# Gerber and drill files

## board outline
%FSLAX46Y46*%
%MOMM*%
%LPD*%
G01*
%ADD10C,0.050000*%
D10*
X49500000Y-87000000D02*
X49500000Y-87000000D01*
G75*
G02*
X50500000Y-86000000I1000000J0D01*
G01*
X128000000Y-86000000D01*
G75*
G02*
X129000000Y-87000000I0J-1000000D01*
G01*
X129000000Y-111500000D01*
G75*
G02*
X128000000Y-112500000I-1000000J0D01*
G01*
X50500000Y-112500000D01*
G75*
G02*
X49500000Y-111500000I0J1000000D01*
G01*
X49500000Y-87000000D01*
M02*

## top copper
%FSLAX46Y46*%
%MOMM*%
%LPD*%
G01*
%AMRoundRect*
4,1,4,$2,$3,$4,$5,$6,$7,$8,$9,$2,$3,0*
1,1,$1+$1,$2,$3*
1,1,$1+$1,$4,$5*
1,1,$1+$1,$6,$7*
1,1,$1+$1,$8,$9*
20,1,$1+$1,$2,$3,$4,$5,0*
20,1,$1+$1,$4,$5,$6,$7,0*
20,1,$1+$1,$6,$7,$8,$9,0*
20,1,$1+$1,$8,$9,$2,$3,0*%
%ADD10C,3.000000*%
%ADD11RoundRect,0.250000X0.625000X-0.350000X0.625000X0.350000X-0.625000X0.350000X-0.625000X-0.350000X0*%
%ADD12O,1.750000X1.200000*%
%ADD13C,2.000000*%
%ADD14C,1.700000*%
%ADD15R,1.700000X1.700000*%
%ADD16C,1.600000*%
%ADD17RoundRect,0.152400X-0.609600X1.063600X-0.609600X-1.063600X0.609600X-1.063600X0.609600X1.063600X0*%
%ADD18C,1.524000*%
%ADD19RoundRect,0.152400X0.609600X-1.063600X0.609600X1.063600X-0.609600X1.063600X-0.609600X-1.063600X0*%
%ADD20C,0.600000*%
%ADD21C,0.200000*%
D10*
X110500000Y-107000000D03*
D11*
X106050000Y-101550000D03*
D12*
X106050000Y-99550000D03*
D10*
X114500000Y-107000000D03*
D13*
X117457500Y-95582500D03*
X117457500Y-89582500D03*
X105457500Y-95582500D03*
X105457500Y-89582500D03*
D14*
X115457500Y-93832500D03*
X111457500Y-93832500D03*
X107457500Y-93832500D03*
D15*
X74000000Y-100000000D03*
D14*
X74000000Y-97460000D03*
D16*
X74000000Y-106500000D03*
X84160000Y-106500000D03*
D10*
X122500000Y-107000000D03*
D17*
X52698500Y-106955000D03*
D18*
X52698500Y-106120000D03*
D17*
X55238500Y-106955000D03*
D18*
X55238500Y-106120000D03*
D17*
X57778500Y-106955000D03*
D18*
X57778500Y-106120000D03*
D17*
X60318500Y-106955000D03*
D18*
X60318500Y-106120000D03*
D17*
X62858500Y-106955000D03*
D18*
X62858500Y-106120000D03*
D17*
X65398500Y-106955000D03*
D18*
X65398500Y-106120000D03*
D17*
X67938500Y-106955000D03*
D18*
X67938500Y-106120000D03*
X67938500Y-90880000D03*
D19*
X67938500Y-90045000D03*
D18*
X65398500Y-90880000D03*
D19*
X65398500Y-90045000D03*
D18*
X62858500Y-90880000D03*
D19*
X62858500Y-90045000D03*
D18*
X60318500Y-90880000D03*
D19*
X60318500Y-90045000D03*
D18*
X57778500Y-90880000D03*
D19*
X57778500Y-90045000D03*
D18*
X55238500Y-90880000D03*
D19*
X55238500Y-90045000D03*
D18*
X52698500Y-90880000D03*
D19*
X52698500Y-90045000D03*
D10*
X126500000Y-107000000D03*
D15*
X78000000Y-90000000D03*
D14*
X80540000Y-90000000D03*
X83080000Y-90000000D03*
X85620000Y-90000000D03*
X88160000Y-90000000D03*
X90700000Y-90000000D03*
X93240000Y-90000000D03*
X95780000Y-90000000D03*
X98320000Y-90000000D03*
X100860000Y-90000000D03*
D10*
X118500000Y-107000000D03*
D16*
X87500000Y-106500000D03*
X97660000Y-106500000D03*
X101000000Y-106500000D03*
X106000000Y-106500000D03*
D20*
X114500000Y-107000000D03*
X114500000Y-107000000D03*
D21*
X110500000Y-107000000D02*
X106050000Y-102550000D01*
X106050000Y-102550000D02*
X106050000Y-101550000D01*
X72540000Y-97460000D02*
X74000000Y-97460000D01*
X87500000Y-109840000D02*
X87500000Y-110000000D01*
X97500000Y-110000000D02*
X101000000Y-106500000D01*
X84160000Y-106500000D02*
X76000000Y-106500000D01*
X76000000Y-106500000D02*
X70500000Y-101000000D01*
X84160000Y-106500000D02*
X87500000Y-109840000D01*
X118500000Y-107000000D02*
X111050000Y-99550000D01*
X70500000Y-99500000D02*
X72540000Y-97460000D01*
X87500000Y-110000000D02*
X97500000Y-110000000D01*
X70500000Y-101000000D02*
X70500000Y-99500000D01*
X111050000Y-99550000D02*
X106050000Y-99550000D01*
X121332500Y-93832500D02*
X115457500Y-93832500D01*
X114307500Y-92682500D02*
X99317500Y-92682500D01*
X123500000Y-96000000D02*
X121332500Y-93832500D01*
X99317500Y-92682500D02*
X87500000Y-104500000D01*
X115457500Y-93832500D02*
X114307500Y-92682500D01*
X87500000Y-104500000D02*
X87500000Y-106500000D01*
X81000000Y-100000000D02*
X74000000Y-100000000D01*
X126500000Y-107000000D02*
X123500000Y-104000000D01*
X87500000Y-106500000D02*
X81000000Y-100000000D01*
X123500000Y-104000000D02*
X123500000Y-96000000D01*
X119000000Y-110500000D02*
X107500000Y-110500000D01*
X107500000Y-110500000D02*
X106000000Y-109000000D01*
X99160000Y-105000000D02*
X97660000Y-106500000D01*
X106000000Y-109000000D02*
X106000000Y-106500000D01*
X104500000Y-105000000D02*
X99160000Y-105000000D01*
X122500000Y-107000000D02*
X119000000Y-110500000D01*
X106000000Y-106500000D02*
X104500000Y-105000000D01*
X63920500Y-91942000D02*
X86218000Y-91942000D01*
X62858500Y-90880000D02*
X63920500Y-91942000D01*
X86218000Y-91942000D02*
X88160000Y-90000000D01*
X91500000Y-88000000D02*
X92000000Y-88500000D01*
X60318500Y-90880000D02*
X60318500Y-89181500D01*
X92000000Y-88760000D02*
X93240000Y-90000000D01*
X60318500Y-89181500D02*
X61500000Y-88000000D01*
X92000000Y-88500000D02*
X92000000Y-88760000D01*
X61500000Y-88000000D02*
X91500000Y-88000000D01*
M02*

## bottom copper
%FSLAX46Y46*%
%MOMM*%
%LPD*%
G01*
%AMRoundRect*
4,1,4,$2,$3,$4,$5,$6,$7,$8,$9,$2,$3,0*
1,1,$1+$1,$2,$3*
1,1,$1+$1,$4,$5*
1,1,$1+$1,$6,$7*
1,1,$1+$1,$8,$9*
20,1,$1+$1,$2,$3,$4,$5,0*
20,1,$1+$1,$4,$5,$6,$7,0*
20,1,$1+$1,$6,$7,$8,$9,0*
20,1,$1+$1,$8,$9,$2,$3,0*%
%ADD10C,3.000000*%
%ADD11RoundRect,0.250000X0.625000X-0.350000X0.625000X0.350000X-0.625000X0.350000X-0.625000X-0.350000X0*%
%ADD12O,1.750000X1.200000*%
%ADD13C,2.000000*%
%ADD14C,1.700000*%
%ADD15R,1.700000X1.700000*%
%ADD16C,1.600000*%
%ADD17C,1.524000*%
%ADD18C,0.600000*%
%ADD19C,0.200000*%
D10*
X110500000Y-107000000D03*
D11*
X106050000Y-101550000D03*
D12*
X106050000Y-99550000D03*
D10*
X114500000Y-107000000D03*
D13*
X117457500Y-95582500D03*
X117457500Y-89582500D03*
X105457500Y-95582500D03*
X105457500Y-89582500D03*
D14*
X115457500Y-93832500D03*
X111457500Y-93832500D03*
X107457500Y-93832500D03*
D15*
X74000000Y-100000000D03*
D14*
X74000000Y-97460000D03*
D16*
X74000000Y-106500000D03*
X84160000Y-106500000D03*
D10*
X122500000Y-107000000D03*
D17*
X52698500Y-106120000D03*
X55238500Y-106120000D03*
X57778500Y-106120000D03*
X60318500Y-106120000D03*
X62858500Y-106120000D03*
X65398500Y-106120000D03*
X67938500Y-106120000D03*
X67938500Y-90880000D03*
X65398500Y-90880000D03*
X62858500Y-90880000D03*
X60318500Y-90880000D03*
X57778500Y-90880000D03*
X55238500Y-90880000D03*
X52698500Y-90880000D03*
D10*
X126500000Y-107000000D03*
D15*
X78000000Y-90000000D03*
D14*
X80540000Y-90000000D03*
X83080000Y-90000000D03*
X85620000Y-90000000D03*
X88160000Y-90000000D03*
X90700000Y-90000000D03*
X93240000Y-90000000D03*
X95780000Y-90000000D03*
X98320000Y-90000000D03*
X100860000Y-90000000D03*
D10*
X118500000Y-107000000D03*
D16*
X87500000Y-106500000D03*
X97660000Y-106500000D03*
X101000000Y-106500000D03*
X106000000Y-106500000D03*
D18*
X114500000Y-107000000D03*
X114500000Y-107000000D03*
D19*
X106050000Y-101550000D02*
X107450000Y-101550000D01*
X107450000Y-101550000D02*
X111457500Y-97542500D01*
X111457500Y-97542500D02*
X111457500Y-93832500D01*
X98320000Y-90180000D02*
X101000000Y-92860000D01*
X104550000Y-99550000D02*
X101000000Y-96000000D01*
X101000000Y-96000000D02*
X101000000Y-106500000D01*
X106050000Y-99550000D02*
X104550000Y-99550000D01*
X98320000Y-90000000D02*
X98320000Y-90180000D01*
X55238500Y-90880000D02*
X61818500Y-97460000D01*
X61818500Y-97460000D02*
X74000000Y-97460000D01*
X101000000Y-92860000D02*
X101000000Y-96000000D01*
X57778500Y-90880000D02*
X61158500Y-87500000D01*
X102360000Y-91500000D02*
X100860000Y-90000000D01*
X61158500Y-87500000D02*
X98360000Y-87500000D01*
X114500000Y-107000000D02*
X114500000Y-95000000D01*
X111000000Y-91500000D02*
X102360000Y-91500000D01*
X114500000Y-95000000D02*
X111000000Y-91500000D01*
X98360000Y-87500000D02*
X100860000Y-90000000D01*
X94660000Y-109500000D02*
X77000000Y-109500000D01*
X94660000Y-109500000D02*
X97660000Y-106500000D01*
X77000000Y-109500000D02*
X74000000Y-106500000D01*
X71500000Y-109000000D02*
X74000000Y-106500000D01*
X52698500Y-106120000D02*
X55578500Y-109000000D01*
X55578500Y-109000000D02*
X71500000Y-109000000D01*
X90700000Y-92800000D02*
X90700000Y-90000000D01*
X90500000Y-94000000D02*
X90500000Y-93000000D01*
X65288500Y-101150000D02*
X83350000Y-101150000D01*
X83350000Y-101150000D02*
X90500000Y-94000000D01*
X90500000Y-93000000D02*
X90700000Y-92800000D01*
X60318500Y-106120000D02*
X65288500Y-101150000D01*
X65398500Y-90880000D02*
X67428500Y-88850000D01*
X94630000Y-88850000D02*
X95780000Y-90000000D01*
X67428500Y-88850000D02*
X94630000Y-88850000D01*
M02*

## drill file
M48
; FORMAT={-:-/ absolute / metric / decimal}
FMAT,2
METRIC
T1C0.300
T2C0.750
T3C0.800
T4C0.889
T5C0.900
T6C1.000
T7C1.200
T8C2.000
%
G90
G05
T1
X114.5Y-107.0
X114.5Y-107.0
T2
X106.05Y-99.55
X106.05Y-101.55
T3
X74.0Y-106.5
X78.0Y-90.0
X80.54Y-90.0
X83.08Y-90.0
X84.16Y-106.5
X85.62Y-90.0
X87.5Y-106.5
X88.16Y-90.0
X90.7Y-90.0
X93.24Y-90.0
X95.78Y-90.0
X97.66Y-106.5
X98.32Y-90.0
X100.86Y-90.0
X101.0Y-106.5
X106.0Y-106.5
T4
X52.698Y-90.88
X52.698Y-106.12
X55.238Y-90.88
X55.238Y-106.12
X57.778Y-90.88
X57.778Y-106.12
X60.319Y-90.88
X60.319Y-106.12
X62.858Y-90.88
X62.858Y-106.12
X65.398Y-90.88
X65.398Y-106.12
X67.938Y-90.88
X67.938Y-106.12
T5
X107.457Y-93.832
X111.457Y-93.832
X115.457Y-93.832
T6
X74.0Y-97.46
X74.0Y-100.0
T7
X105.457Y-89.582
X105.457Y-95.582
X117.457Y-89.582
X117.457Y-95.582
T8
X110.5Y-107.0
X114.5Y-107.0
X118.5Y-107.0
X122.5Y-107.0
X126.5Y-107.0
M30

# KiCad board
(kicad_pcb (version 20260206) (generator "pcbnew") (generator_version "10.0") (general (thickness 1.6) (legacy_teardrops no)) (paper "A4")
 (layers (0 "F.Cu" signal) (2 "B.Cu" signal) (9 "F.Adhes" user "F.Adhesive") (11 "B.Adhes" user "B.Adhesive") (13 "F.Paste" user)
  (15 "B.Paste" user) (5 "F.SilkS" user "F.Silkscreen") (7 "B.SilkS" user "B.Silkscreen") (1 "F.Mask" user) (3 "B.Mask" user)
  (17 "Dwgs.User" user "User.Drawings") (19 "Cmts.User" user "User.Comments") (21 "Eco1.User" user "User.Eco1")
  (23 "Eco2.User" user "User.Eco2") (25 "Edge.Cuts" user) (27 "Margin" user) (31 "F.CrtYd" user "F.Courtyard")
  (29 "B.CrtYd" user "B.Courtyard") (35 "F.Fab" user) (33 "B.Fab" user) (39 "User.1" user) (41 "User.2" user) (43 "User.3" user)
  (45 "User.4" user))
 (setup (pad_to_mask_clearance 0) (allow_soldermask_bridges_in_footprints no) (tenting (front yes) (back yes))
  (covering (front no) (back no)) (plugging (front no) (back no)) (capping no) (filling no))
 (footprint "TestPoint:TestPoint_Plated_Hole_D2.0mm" (layer "F.Cu") (at 110.5 107)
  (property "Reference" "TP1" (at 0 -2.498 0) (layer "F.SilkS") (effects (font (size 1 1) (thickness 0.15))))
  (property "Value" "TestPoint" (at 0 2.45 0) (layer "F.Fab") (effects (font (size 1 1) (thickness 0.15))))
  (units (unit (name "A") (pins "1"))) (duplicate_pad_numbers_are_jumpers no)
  (pad "1" thru_hole circle (at 0 0) (size 3 3) (drill 2) (layers "*.Cu" "*.Mask") (remove_unused_layers no) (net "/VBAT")))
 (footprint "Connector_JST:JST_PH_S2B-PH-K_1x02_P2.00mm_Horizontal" (layer "F.Cu") (at 106.05 101.55 90)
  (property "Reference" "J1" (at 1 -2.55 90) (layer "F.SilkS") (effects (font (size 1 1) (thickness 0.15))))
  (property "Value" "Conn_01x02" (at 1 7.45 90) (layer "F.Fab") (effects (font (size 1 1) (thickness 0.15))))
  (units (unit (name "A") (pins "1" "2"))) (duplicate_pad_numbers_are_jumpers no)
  (pad "1" thru_hole roundrect (at 0 0 90) (size 1.2 1.75) (drill 0.75) (layers "*.Cu" "*.Mask") (remove_unused_layers no)
   (roundrect_rratio 0.208333) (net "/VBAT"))
  (pad "2" thru_hole oval (at 2 0 90) (size 1.2 1.75) (drill 0.75) (layers "*.Cu" "*.Mask") (remove_unused_layers no) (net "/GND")))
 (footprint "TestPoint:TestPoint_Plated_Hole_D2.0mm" (layer "F.Cu") (at 114.5 107)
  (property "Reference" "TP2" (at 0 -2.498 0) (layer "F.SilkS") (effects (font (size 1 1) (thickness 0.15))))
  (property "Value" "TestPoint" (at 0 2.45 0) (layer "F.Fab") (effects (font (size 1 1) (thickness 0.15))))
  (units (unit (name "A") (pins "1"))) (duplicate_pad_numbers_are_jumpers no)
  (pad "1" thru_hole circle (at 0 0) (size 3 3) (drill 2) (layers "*.Cu" "*.Mask") (remove_unused_layers no) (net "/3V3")))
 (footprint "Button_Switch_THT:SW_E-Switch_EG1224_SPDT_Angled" (layer "F.Cu") (at 115.4575 93.8325 180)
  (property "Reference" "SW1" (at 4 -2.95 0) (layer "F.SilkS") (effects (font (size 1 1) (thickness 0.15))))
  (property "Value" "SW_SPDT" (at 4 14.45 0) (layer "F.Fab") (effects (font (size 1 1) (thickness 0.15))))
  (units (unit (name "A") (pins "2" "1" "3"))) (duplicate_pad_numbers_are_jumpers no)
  (pad "" thru_hole circle (at -2 -1.75 180) (size 2 2) (drill 1.2) (layers "*.Cu" "*.Mask") (remove_unused_layers no))
  (pad "" thru_hole circle (at -2 4.25 180) (size 2 2) (drill 1.2) (layers "*.Cu" "*.Mask") (remove_unused_layers no))
  (pad "" thru_hole circle (at 10 -1.75 180) (size 2 2) (drill 1.2) (layers "*.Cu" "*.Mask") (remove_unused_layers no))
  (pad "" thru_hole circle (at 10 4.25 180) (size 2 2) (drill 1.2) (layers "*.Cu" "*.Mask") (remove_unused_layers no))
  (pad "1" thru_hole circle (at 0 0 180) (size 1.7 1.7) (drill 0.9) (layers "*.Cu" "*.Mask") (remove_unused_layers no)
   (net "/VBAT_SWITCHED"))
  (pad "2" thru_hole circle (at 4 0 180) (size 1.7 1.7) (drill 0.9) (layers "*.Cu" "*.Mask") (remove_unused_layers no) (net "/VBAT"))
  (pad "3" thru_hole circle (at 8 0 180) (size 1.7 1.7) (drill 0.9) (layers "*.Cu" "*.Mask") (remove_unused_layers no)
   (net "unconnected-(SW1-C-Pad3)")))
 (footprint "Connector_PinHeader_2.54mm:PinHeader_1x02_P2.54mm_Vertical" (layer "F.Cu") (at 74 100 180)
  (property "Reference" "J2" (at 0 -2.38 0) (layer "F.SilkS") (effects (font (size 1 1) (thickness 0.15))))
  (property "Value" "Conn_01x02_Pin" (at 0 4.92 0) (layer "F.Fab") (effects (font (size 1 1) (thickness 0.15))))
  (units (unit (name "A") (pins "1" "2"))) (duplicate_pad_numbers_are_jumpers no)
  (pad "1" thru_hole rect (at 0 0 180) (size 1.7 1.7) (drill 1) (layers "*.Cu" "*.Mask") (remove_unused_layers no) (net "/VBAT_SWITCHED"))
  (pad "2" thru_hole circle (at 0 2.54 180) (size 1.7 1.7) (drill 1) (layers "*.Cu" "*.Mask") (remove_unused_layers no) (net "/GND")))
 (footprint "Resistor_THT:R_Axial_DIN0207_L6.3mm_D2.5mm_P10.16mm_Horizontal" (layer "F.Cu") (at 74 106.5)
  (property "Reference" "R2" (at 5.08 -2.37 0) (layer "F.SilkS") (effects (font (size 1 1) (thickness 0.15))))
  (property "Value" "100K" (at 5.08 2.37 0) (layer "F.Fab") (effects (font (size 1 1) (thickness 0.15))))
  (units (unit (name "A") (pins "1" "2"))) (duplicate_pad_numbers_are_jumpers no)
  (pad "1" thru_hole circle (at 0 0) (size 1.6 1.6) (drill 0.8) (layers "*.Cu" "*.Mask") (remove_unused_layers no) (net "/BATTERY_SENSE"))
  (pad "2" thru_hole circle (at 10.16 0) (size 1.6 1.6) (drill 0.8) (layers "*.Cu" "*.Mask") (remove_unused_layers no) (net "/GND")))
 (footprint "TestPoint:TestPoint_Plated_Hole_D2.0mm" (layer "F.Cu") (at 122.5 107)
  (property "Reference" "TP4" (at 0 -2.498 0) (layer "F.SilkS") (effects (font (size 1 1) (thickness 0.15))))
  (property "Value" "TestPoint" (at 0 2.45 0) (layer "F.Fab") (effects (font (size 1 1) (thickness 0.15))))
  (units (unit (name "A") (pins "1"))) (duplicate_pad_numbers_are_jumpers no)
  (pad "1" thru_hole circle (at 0 0) (size 3 3) (drill 2) (layers "*.Cu" "*.Mask") (remove_unused_layers no) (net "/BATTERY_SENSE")))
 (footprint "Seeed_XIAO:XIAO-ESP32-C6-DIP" (layer "F.Cu") (at 60.3185 98.5 180)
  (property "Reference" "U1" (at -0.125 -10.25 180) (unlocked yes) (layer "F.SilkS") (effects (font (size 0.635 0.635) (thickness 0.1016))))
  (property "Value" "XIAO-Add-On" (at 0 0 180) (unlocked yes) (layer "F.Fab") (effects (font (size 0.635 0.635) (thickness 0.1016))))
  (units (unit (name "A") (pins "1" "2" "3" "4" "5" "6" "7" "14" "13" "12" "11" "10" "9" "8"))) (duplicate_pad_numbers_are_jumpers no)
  (pad "1" smd roundrect (at 7.62 -8.455 270) (size 2.432 1.524) (layers "F.Cu" "F.Mask") (roundrect_rratio 0.1) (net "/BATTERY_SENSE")
   (thermal_bridge_angle 45))
  (pad "1" thru_hole circle (at 7.62 -7.62 270) (size 1.524 1.524) (drill 0.889) (layers "*.Cu" "*.Mask") (remove_unused_layers no)
   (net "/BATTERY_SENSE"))
  (pad "2" smd roundrect (at 5.08 -8.455 270) (size 2.432 1.524) (layers "F.Cu" "F.Mask") (roundrect_rratio 0.1)
   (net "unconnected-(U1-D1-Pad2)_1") (thermal_bridge_angle 45))
  (pad "2" thru_hole circle (at 5.08 -7.62 270) (size 1.524 1.524) (drill 0.889) (layers "*.Cu" "*.Mask") (remove_unused_layers no)
   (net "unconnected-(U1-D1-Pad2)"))
  (pad "3" smd roundrect (at 2.54 -8.455 270) (size 2.432 1.524) (layers "F.Cu" "F.Mask") (roundrect_rratio 0.1)
   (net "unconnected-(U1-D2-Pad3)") (thermal_bridge_angle 45))
  (pad "3" thru_hole circle (at 2.54 -7.62 270) (size 1.524 1.524) (drill 0.889) (layers "*.Cu" "*.Mask") (remove_unused_layers no)
   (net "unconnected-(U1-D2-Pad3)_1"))
  (pad "4" smd roundrect (at 0 -8.455 270) (size 2.432 1.524) (layers "F.Cu" "F.Mask") (roundrect_rratio 0.1) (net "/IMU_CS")
   (thermal_bridge_angle 45))
  (pad "4" thru_hole circle (at 0 -7.62 270) (size 1.524 1.524) (drill 0.889) (layers "*.Cu" "*.Mask") (remove_unused_layers no)
   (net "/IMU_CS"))
  (pad "5" smd roundrect (at -2.54 -8.455 270) (size 2.432 1.524) (layers "F.Cu" "F.Mask") (roundrect_rratio 0.1)
   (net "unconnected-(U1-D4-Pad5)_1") (thermal_bridge_angle 45))
  (pad "5" thru_hole circle (at -2.54 -7.62 270) (size 1.524 1.524) (drill 0.889) (layers "*.Cu" "*.Mask") (remove_unused_layers no)
   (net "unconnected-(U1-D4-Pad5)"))
  (pad "6" smd roundrect (at -5.08 -8.455 270) (size 2.432 1.524) (layers "F.Cu" "F.Mask") (roundrect_rratio 0.1)
   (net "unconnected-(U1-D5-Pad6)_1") (thermal_bridge_angle 45))
  (pad "6" thru_hole circle (at -5.08 -7.62 270) (size 1.524 1.524) (drill 0.889) (layers "*.Cu" "*.Mask") (remove_unused_layers no)
   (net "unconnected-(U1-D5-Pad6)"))
  (pad "7" smd roundrect (at -7.62 -8.455 270) (size 2.432 1.524) (layers "F.Cu" "F.Mask") (roundrect_rratio 0.1)
   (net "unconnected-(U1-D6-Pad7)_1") (thermal_bridge_angle 45))
  (pad "7" thru_hole circle (at -7.62 -7.62 270) (size 1.524 1.524) (drill 0.889) (layers "*.Cu" "*.Mask") (remove_unused_layers no)
   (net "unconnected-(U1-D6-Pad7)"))
  (pad "8" thru_hole circle (at -7.62 7.62 90) (size 1.524 1.524) (drill 0.889) (layers "*.Cu" "*.Mask") (remove_unused_layers no)
   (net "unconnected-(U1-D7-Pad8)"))
  (pad "8" smd roundrect (at -7.62 8.455 90) (size 2.432 1.524) (layers "F.Cu" "F.Mask") (roundrect_rratio 0.1)
   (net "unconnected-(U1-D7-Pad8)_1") (thermal_bridge_angle 45))
  (pad "9" thru_hole circle (at -5.08 7.62 90) (size 1.524 1.524) (drill 0.889) (layers "*.Cu" "*.Mask") (remove_unused_layers no)
   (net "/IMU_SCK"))
  (pad "9" smd roundrect (at -5.08 8.455 90) (size 2.432 1.524) (layers "F.Cu" "F.Mask") (roundrect_rratio 0.1) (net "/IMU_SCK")
   (thermal_bridge_angle 45))
  (pad "10" thru_hole circle (at -2.54 7.62 90) (size 1.524 1.524) (drill 0.889) (layers "*.Cu" "*.Mask") (remove_unused_layers no)
   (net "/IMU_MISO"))
  (pad "10" smd roundrect (at -2.54 8.455 90) (size 2.432 1.524) (layers "F.Cu" "F.Mask") (roundrect_rratio 0.1) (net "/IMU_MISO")
   (thermal_bridge_angle 45))
  (pad "11" thru_hole circle (at 0 7.62 90) (size 1.524 1.524) (drill 0.889) (layers "*.Cu" "*.Mask") (remove_unused_layers no)
   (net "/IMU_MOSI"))
  (pad "11" smd roundrect (at 0 8.455 90) (size 2.432 1.524) (layers "F.Cu" "F.Mask") (roundrect_rratio 0.1) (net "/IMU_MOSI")
   (thermal_bridge_angle 45))
  (pad "12" thru_hole circle (at 2.54 7.62 90) (size 1.524 1.524) (drill 0.889) (layers "*.Cu" "*.Mask") (remove_unused_layers no)
   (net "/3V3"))
  (pad "12" smd roundrect (at 2.54 8.455 90) (size 2.432 1.524) (layers "F.Cu" "F.Mask") (roundrect_rratio 0.1) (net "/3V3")
   (thermal_bridge_angle 45))
  (pad "13" thru_hole circle (at 5.08 7.62 90) (size 1.524 1.524) (drill 0.889) (layers "*.Cu" "*.Mask") (remove_unused_layers no)
   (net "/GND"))
  (pad "13" smd roundrect (at 5.08 8.455 90) (size 2.432 1.524) (layers "F.Cu" "F.Mask") (roundrect_rratio 0.1) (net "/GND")
   (thermal_bridge_angle 45))
  (pad "14" thru_hole circle (at 7.62 7.62 90) (size 1.524 1.524) (drill 0.889) (layers "*.Cu" "*.Mask") (remove_unused_layers no)
   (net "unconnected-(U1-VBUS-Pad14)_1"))
  (pad "14" smd roundrect (at 7.62 8.455 90) (size 2.432 1.524) (layers "F.Cu" "F.Mask") (roundrect_rratio 0.1)
   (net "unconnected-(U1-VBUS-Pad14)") (thermal_bridge_angle 45)))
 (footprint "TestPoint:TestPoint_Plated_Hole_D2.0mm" (layer "F.Cu") (at 126.5 107)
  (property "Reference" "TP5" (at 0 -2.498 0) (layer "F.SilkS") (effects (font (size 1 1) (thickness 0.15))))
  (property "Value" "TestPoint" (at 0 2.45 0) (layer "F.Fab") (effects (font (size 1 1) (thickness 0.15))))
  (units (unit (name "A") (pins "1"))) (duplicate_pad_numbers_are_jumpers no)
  (pad "1" thru_hole circle (at 0 0) (size 3 3) (drill 2) (layers "*.Cu" "*.Mask") (remove_unused_layers no) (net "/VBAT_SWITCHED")))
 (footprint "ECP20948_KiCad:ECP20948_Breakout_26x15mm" (layer "F.Cu") (at 77 89)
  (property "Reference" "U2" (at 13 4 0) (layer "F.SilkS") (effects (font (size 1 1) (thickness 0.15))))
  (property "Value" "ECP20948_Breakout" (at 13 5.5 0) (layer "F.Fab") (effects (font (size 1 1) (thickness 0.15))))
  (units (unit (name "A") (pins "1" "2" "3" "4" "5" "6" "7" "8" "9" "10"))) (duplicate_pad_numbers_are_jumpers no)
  (pad "1" thru_hole rect (at 1 1) (size 1.7 1.7) (drill 0.8) (layers "*.Cu" "*.Mask") (remove_unused_layers no)
   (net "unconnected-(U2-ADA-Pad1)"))
  (pad "2" thru_hole circle (at 3.54 1) (size 1.7 1.7) (drill 0.8) (layers "*.Cu" "*.Mask") (remove_unused_layers no)
   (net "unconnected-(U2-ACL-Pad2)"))
  (pad "3" thru_hole circle (at 6.08 1) (size 1.7 1.7) (drill 0.8) (layers "*.Cu" "*.Mask") (remove_unused_layers no)
   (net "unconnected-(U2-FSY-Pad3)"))
  (pad "4" thru_hole circle (at 8.62 1) (size 1.7 1.7) (drill 0.8) (layers "*.Cu" "*.Mask") (remove_unused_layers no)
   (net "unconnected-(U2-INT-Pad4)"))
  (pad "5" thru_hole circle (at 11.16 1) (size 1.7 1.7) (drill 0.8) (layers "*.Cu" "*.Mask") (remove_unused_layers no) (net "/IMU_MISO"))
  (pad "6" thru_hole circle (at 13.7 1) (size 1.7 1.7) (drill 0.8) (layers "*.Cu" "*.Mask") (remove_unused_layers no) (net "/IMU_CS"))
  (pad "7" thru_hole circle (at 16.24 1) (size 1.7 1.7) (drill 0.8) (layers "*.Cu" "*.Mask") (remove_unused_layers no) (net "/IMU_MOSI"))
  (pad "8" thru_hole circle (at 18.78 1) (size 1.7 1.7) (drill 0.8) (layers "*.Cu" "*.Mask") (remove_unused_layers no) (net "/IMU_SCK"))
  (pad "9" thru_hole circle (at 21.32 1) (size 1.7 1.7) (drill 0.8) (layers "*.Cu" "*.Mask") (remove_unused_layers no) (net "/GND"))
  (pad "10" thru_hole circle (at 23.86 1) (size 1.7 1.7) (drill 0.8) (layers "*.Cu" "*.Mask") (remove_unused_layers no) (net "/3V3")))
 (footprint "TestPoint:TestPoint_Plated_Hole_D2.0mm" (layer "F.Cu") (at 118.5 107)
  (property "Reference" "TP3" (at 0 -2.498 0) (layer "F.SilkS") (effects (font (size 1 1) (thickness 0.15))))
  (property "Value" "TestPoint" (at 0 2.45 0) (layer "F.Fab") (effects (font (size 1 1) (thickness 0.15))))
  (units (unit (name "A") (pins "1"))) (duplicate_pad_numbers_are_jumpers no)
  (pad "1" thru_hole circle (at 0 0) (size 3 3) (drill 2) (layers "*.Cu" "*.Mask") (remove_unused_layers no) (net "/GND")))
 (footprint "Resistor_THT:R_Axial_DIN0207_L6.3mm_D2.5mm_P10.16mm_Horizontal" (layer "F.Cu") (at 87.5 106.5)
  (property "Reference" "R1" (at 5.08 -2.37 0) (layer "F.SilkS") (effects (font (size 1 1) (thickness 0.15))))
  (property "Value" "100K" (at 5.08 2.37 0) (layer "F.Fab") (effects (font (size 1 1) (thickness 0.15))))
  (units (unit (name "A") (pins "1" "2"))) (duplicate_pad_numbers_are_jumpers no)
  (pad "1" thru_hole circle (at 0 0) (size 1.6 1.6) (drill 0.8) (layers "*.Cu" "*.Mask") (remove_unused_layers no) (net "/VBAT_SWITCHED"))
  (pad "2" thru_hole circle (at 10.16 0) (size 1.6 1.6) (drill 0.8) (layers "*.Cu" "*.Mask") (remove_unused_layers no)
   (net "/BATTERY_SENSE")))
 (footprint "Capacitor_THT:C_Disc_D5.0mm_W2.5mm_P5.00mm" (layer "F.Cu") (at 101 106.5)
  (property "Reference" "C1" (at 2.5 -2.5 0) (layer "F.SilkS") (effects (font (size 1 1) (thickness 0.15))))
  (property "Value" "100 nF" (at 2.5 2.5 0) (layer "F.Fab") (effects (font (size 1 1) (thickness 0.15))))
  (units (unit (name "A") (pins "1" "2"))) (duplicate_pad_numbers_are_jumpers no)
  (pad "1" thru_hole circle (at 0 0) (size 1.6 1.6) (drill 0.8) (layers "*.Cu" "*.Mask") (remove_unused_layers no) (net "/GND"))
  (pad "2" thru_hole circle (at 5 0) (size 1.6 1.6) (drill 0.8) (layers "*.Cu" "*.Mask") (remove_unused_layers no) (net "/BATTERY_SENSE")))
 (gr_rect (start 49.5 86) (end 129 112.5) (radius 1) (stroke (width 0.05) (type default)) (fill no) (layer "Edge.Cuts"))
 (segment (start 110.5 107) (end 106.05 102.55) (width 0.2) (layer "F.Cu") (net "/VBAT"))
 (segment (start 106.05 102.55) (end 106.05 101.55) (width 0.2) (layer "F.Cu") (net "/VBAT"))
 (segment (start 106.05 101.55) (end 107.45 101.55) (width 0.2) (layer "B.Cu") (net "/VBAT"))
 (segment (start 107.45 101.55) (end 111.4575 97.5425) (width 0.2) (layer "B.Cu") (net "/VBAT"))
 (segment (start 111.4575 97.5425) (end 111.4575 93.8325) (width 0.2) (layer "B.Cu") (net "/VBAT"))
 (segment (start 72.54 97.46) (end 74 97.46) (width 0.2) (layer "F.Cu") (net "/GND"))
 (segment (start 87.5 109.84) (end 87.5 110) (width 0.2) (layer "F.Cu") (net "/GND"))
 (segment (start 97.5 110) (end 101 106.5) (width 0.2) (layer "F.Cu") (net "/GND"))
 (segment (start 84.16 106.5) (end 76 106.5) (width 0.2) (layer "F.Cu") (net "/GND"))
 (segment (start 76 106.5) (end 70.5 101) (width 0.2) (layer "F.Cu") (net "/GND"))
 (segment (start 84.16 106.5) (end 87.5 109.84) (width 0.2) (layer "F.Cu") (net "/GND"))
 (segment (start 118.5 107) (end 111.05 99.55) (width 0.2) (layer "F.Cu") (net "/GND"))
 (segment (start 70.5 99.5) (end 72.54 97.46) (width 0.2) (layer "F.Cu") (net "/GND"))
 (segment (start 87.5 110) (end 97.5 110) (width 0.2) (layer "F.Cu") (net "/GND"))
 (segment (start 70.5 101) (end 70.5 99.5) (width 0.2) (layer "F.Cu") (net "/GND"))
 (segment (start 111.05 99.55) (end 106.05 99.55) (width 0.2) (layer "F.Cu") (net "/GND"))
 (segment (start 98.32 90.18) (end 101 92.86) (width 0.2) (layer "B.Cu") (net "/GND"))
 (segment (start 104.55 99.55) (end 101 96) (width 0.2) (layer "B.Cu") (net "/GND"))
 (segment (start 101 96) (end 101 106.5) (width 0.2) (layer "B.Cu") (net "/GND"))
 (segment (start 106.05 99.55) (end 104.55 99.55) (width 0.2) (layer "B.Cu") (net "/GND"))
 (segment (start 98.32 90) (end 98.32 90.18) (width 0.2) (layer "B.Cu") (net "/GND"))
 (segment (start 55.2385 90.88) (end 61.8185 97.46) (width 0.2) (layer "B.Cu") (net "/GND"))
 (segment (start 61.8185 97.46) (end 74 97.46) (width 0.2) (layer "B.Cu") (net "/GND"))
 (segment (start 101 92.86) (end 101 96) (width 0.2) (layer "B.Cu") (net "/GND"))
 (via (at 114.5 107) (size 0.6) (drill 0.3) (layers "F.Cu" "B.Cu") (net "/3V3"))
 (via (at 114.5 107) (size 0.6) (drill 0.3) (layers "F.Cu" "B.Cu") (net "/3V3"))
 (segment (start 57.7785 90.88) (end 61.1585 87.5) (width 0.2) (layer "B.Cu") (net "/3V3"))
 (segment (start 102.36 91.5) (end 100.86 90) (width 0.2) (layer "B.Cu") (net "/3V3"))
 (segment (start 61.1585 87.5) (end 98.36 87.5) (width 0.2) (layer "B.Cu") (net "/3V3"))
 (segment (start 114.5 107) (end 114.5 95) (width 0.2) (layer "B.Cu") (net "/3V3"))
 (segment (start 111 91.5) (end 102.36 91.5) (width 0.2) (layer "B.Cu") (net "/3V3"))
 (segment (start 114.5 95) (end 111 91.5) (width 0.2) (layer "B.Cu") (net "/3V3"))
 (segment (start 98.36 87.5) (end 100.86 90) (width 0.2) (layer "B.Cu") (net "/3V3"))
 (segment (start 121.3325 93.8325) (end 115.4575 93.8325) (width 0.2) (layer "F.Cu") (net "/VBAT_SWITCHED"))
 (segment (start 114.3075 92.6825) (end 99.3175 92.6825) (width 0.2) (layer "F.Cu") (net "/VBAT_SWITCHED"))
 (segment (start 123.5 96) (end 121.3325 93.8325) (width 0.2) (layer "F.Cu") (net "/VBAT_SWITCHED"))
 (segment (start 99.3175 92.6825) (end 87.5 104.5) (width 0.2) (layer "F.Cu") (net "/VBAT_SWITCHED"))
 (segment (start 115.4575 93.8325) (end 114.3075 92.6825) (width 0.2) (layer "F.Cu") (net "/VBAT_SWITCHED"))
 (segment (start 87.5 104.5) (end 87.5 106.5) (width 0.2) (layer "F.Cu") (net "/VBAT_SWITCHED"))
 (segment (start 81 100) (end 74 100) (width 0.2) (layer "F.Cu") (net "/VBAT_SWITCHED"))
 (segment (start 126.5 107) (end 123.5 104) (width 0.2) (layer "F.Cu") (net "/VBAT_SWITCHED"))
 (segment (start 87.5 106.5) (end 81 100) (width 0.2) (layer "F.Cu") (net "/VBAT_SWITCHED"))
 (segment (start 123.5 104) (end 123.5 96) (width 0.2) (layer "F.Cu") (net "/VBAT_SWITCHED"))
 (segment (start 119 110.5) (end 107.5 110.5) (width 0.2) (layer "F.Cu") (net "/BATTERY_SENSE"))
 (segment (start 107.5 110.5) (end 106 109) (width 0.2) (layer "F.Cu") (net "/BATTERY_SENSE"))
 (segment (start 99.16 105) (end 97.66 106.5) (width 0.2) (layer "F.Cu") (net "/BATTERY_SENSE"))
 (segment (start 106 109) (end 106 106.5) (width 0.2) (layer "F.Cu") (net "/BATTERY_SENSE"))
 (segment (start 104.5 105) (end 99.16 105) (width 0.2) (layer "F.Cu") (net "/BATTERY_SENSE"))
 (segment (start 122.5 107) (end 119 110.5) (width 0.2) (layer "F.Cu") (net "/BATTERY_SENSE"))
 (segment (start 106 106.5) (end 104.5 105) (width 0.2) (layer "F.Cu") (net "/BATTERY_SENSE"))
 (segment (start 94.66 109.5) (end 77 109.5) (width 0.2) (layer "B.Cu") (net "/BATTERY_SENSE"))
 (segment (start 94.66 109.5) (end 97.66 106.5) (width 0.2) (layer "B.Cu") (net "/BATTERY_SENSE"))
 (segment (start 77 109.5) (end 74 106.5) (width 0.2) (layer "B.Cu") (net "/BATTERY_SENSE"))
 (segment (start 71.5 109) (end 74 106.5) (width 0.2) (layer "B.Cu") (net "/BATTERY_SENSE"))
 (segment (start 52.6985 106.12) (end 55.5785 109) (width 0.2) (layer "B.Cu") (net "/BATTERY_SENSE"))
 (segment (start 55.5785 109) (end 71.5 109) (width 0.2) (layer "B.Cu") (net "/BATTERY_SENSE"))
 (segment (start 90.7 92.8) (end 90.7 90) (width 0.2) (layer "B.Cu") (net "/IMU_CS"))
 (segment (start 90.5 94) (end 90.5 93) (width 0.2) (layer "B.Cu") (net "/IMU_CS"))
 (segment (start 65.2885 101.15) (end 83.35 101.15) (width 0.2) (layer "B.Cu") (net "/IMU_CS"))
 (segment (start 83.35 101.15) (end 90.5 94) (width 0.2) (layer "B.Cu") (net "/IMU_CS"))
 (segment (start 90.5 93) (end 90.7 92.8) (width 0.2) (layer "B.Cu") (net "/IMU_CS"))
 (segment (start 60.3185 106.12) (end 65.2885 101.15) (width 0.2) (layer "B.Cu") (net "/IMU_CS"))
 (segment (start 65.3985 90.88) (end 67.4285 88.85) (width 0.2) (layer "B.Cu") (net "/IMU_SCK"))
 (segment (start 94.63 88.85) (end 95.78 90) (width 0.2) (layer "B.Cu") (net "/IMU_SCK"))
 (segment (start 67.4285 88.85) (end 94.63 88.85) (width 0.2) (layer "B.Cu") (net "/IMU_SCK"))
 (segment (start 63.9205 91.942) (end 86.218 91.942) (width 0.2) (layer "F.Cu") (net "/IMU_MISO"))
 (segment (start 62.8585 90.88) (end 63.9205 91.942) (width 0.2) (layer "F.Cu") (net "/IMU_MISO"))
 (segment (start 86.218 91.942) (end 88.16 90) (width 0.2) (layer "F.Cu") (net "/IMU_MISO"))
 (segment (start 91.5 88) (end 92 88.5) (width 0.2) (layer "F.Cu") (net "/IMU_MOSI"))
 (segment (start 60.3185 90.88) (end 60.3185 89.1815) (width 0.2) (layer "F.Cu") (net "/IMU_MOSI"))
 (segment (start 92 88.76) (end 93.24 90) (width 0.2) (layer "F.Cu") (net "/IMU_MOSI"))
 (segment (start 60.3185 89.1815) (end 61.5 88) (width 0.2) (layer "F.Cu") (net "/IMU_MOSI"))
 (segment (start 92 88.5) (end 92 88.76) (width 0.2) (layer "F.Cu") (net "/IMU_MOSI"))
 (segment (start 61.5 88) (end 91.5 88) (width 0.2) (layer "F.Cu") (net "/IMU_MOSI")))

